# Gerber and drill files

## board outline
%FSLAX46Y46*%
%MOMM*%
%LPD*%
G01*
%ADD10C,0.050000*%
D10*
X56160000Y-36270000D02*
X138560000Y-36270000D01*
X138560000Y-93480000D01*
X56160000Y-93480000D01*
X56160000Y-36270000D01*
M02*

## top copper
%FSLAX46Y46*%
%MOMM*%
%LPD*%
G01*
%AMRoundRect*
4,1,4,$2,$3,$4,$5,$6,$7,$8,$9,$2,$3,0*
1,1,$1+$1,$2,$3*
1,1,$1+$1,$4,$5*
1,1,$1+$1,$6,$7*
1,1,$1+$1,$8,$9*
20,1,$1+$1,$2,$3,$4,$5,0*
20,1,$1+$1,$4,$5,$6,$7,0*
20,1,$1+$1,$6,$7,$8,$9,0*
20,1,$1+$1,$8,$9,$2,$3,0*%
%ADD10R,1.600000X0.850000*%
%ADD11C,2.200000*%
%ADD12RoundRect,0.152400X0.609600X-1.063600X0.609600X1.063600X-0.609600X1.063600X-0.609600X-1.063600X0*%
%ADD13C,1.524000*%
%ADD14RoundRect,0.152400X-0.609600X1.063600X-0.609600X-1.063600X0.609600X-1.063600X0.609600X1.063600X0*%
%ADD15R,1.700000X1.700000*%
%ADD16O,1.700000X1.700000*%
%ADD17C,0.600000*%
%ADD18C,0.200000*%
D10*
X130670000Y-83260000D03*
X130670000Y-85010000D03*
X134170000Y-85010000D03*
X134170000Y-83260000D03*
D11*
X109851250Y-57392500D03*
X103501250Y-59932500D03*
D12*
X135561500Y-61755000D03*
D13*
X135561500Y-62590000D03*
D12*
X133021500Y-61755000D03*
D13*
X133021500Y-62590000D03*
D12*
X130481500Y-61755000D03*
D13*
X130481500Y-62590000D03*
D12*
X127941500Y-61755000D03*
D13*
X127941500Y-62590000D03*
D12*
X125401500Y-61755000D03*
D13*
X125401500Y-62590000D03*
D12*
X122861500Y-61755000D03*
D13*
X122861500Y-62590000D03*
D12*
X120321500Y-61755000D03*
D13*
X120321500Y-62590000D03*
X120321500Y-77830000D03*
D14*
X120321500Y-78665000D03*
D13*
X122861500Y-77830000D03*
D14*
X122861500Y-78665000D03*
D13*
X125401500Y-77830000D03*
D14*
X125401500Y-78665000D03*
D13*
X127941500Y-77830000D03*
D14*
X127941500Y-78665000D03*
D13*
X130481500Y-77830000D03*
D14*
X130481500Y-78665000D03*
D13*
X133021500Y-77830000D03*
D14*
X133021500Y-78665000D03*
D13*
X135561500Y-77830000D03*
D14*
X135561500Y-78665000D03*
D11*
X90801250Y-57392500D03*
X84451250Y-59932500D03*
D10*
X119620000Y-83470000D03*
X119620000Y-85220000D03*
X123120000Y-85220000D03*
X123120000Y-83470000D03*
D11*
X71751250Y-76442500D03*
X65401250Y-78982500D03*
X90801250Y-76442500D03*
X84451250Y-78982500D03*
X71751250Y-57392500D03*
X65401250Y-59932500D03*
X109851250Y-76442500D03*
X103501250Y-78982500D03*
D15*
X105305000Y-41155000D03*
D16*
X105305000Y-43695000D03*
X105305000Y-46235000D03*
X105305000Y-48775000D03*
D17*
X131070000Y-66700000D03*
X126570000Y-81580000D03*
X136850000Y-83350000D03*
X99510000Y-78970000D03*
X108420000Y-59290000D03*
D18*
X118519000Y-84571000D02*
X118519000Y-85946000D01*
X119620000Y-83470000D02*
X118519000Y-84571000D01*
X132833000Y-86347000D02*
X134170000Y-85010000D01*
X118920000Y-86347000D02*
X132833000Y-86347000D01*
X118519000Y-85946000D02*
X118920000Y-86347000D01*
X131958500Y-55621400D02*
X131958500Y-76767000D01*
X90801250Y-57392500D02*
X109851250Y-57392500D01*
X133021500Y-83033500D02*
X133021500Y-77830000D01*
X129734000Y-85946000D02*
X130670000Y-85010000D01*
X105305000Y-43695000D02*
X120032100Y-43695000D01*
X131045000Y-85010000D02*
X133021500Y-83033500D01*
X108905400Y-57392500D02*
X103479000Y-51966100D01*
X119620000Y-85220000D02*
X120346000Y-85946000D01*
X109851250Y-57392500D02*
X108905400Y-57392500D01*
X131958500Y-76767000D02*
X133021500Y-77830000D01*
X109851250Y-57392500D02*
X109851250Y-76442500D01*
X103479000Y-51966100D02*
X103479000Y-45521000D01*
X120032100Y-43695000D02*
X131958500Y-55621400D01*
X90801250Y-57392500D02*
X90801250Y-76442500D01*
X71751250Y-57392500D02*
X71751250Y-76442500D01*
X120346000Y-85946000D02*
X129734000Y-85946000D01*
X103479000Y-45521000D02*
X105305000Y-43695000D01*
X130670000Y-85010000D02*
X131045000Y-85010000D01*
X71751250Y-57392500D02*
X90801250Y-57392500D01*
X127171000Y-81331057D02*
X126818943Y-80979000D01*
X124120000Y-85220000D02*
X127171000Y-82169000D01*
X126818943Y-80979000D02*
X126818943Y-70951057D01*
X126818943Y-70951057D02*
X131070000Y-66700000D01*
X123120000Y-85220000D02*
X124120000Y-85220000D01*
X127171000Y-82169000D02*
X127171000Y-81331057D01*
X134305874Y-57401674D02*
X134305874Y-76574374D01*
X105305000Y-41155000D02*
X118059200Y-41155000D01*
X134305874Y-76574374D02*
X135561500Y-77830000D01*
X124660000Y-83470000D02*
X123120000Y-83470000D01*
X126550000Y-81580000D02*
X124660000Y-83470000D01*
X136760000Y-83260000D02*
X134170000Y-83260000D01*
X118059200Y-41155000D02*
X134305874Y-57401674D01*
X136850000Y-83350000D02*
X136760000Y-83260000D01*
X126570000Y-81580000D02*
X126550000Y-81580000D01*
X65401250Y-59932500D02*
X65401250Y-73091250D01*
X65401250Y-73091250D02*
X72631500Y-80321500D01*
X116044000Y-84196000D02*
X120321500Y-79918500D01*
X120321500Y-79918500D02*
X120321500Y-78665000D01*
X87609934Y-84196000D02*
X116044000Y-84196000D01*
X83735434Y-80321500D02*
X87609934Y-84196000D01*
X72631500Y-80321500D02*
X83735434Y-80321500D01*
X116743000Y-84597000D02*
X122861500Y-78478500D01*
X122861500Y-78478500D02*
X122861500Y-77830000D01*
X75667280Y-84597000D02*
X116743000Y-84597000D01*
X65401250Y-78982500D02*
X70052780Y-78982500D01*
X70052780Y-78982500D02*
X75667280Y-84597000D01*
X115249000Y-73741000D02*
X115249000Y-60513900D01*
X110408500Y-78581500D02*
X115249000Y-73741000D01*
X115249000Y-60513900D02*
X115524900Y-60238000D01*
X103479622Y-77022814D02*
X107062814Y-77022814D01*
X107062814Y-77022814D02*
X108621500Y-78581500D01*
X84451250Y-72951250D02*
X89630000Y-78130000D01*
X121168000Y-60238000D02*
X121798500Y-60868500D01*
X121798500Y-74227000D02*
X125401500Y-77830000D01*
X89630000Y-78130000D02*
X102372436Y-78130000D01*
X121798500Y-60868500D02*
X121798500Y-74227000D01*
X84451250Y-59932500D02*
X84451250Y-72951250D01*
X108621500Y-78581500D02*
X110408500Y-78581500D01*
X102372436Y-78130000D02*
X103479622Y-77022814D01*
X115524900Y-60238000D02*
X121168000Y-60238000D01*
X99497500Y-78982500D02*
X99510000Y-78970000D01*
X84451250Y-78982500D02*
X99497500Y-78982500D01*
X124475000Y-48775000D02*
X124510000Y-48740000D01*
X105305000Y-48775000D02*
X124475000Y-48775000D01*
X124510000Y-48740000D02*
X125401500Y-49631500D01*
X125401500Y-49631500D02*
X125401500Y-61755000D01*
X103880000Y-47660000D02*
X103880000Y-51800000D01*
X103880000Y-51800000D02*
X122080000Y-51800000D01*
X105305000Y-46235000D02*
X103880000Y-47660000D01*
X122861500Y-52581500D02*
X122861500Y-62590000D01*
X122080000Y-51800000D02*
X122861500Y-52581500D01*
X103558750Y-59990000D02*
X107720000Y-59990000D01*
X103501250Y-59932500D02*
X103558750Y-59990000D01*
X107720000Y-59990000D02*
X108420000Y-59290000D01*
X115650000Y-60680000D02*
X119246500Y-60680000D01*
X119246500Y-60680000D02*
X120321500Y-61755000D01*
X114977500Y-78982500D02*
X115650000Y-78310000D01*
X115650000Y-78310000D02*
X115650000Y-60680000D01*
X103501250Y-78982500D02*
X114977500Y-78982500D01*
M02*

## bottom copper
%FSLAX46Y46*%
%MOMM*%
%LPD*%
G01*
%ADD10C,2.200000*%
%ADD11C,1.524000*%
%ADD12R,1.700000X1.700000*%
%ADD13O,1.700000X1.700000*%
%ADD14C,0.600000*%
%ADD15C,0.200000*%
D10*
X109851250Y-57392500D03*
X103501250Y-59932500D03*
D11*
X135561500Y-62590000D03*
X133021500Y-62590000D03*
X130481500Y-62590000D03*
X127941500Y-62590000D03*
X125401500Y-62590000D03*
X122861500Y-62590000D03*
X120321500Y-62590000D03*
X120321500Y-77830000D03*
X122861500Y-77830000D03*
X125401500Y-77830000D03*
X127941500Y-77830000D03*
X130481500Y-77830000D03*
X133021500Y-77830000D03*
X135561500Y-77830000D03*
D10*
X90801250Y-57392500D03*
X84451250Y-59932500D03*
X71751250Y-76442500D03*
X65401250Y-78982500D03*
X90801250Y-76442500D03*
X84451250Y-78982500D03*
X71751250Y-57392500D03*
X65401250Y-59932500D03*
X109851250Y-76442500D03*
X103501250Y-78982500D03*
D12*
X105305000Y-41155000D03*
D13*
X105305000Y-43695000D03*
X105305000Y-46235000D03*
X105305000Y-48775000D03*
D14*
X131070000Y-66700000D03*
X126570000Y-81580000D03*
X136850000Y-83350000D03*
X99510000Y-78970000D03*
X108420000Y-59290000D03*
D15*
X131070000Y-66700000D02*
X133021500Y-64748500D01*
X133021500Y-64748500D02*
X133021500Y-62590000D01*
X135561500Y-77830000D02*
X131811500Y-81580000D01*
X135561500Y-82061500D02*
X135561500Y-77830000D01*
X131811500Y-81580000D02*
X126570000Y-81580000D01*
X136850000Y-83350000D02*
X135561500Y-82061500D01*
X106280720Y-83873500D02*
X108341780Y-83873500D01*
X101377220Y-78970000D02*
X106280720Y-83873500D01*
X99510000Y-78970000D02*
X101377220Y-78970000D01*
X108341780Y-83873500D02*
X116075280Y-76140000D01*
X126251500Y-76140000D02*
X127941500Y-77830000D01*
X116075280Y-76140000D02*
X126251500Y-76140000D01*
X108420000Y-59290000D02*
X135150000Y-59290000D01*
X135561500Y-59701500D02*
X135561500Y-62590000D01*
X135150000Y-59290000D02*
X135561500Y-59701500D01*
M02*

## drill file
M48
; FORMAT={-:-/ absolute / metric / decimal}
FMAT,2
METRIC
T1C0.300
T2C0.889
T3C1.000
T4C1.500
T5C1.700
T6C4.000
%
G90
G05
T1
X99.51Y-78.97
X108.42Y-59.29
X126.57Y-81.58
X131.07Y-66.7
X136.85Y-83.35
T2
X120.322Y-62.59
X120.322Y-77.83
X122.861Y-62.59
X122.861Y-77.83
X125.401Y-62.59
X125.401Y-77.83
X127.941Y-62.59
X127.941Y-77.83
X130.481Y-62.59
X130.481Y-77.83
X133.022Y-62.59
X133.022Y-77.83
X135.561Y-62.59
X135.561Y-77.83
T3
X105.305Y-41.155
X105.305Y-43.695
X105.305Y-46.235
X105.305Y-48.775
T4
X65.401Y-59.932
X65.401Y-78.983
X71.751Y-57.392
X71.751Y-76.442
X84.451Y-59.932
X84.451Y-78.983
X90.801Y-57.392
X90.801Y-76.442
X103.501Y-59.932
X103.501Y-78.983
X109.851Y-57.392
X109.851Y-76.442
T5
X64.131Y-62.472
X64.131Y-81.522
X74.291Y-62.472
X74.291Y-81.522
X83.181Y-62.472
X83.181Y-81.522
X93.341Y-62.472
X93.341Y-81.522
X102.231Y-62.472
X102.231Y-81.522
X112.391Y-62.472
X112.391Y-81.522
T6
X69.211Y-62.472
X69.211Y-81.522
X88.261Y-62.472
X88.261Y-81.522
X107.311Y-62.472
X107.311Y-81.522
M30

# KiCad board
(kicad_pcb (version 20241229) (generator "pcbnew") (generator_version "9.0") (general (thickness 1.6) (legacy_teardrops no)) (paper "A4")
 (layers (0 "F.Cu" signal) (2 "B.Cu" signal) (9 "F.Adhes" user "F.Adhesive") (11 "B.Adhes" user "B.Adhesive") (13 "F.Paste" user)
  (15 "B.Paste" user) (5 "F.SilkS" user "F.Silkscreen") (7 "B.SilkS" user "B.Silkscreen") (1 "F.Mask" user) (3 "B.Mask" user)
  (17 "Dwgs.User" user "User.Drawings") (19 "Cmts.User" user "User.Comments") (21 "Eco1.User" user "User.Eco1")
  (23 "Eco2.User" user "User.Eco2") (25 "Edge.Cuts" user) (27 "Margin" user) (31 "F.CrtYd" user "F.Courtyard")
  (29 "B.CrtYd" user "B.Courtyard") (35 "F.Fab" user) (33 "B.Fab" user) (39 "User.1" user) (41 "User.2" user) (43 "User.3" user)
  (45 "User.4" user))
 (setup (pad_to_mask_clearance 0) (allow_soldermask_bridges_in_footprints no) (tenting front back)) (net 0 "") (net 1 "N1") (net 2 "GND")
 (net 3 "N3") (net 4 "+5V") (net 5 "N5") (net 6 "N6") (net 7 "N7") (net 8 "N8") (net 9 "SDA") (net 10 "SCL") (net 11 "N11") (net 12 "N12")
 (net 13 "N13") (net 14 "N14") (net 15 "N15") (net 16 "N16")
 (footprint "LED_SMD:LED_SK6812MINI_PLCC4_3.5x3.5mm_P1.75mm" (layer "F.Cu") (at 132.42 84.135)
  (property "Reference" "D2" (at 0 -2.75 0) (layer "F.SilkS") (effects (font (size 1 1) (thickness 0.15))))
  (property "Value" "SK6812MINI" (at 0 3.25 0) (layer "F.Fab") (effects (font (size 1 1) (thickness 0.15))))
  (pad "1" smd rect (at -1.75 -0.875) (size 1.6 0.85) (layers "F.Cu" "F.Mask" "F.Paste") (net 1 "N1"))
  (pad "2" smd rect (at -1.75 0.875) (size 1.6 0.85) (layers "F.Cu" "F.Mask" "F.Paste") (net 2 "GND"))
  (pad "3" smd rect (at 1.75 0.875) (size 1.6 0.85) (layers "F.Cu" "F.Mask" "F.Paste") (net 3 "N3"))
  (pad "4" smd rect (at 1.75 -0.875) (size 1.6 0.85) (layers "F.Cu" "F.Mask" "F.Paste") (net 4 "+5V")))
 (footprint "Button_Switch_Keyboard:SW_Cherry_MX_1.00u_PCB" (layer "F.Cu") (at 109.85125 57.3925)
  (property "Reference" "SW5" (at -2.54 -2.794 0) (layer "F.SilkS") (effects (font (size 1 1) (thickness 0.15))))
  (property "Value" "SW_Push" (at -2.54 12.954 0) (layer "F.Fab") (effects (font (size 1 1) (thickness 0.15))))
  (pad "" np_thru_hole circle (at -7.62 5.08) (size 1.7 1.7) (drill 1.7) (layers "*.Cu" "*.Mask"))
  (pad "" np_thru_hole circle (at -2.54 5.08) (size 4 4) (drill 4) (layers "*.Cu" "*.Mask"))
  (pad "" np_thru_hole circle (at 2.54 5.08) (size 1.7 1.7) (drill 1.7) (layers "*.Cu" "*.Mask"))
  (pad "1" thru_hole circle (at 0 0) (size 2.2 2.2) (drill 1.5) (layers "*.Cu" "*.Mask") (remove_unused_layers no) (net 2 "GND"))
  (pad "2" thru_hole circle (at -6.35 2.54) (size 2.2 2.2) (drill 1.5) (layers "*.Cu" "*.Mask") (remove_unused_layers no) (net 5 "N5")))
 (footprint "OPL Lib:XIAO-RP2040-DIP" (layer "F.Cu") (at 127.9415 70.21 -90)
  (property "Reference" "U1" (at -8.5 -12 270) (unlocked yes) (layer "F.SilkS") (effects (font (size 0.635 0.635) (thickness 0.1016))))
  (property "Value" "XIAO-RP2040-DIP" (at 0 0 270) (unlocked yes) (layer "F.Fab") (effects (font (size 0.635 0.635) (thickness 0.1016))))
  (pad "1" smd roundrect (at -8.455 -7.62 90) (size 2.432 1.524) (layers "F.Cu" "F.Mask") (roundrect_rratio 0.1) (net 5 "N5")
   (thermal_bridge_angle 45))
  (pad "1" thru_hole circle (at -7.62 -7.62 90) (size 1.524 1.524) (drill 0.889) (layers "*.Cu" "*.Mask") (remove_unused_layers no)
   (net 5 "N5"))
  (pad "2" smd roundrect (at -8.455 -5.08 90) (size 2.432 1.524) (layers "F.Cu" "F.Mask") (roundrect_rratio 0.1) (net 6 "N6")
   (thermal_bridge_angle 45))
  (pad "2" thru_hole circle (at -7.62 -5.08 90) (size 1.524 1.524) (drill 0.889) (layers "*.Cu" "*.Mask") (remove_unused_layers no)
   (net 6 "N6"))
  (pad "3" smd roundrect (at -8.455 -2.54 90) (size 2.432 1.524) (layers "F.Cu" "F.Mask") (roundrect_rratio 0.1) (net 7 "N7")
   (thermal_bridge_angle 45))
  (pad "3" thru_hole circle (at -7.62 -2.54 90) (size 1.524 1.524) (drill 0.889) (layers "*.Cu" "*.Mask") (remove_unused_layers no)
   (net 7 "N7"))
  (pad "4" smd roundrect (at -8.455 0 90) (size 2.432 1.524) (layers "F.Cu" "F.Mask") (roundrect_rratio 0.1) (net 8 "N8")
   (thermal_bridge_angle 45))
  (pad "4" thru_hole circle (at -7.62 0 90) (size 1.524 1.524) (drill 0.889) (layers "*.Cu" "*.Mask") (remove_unused_layers no) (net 8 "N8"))
  (pad "5" smd roundrect (at -8.455 2.54 90) (size 2.432 1.524) (layers "F.Cu" "F.Mask") (roundrect_rratio 0.1) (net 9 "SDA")
   (thermal_bridge_angle 45))
  (pad "5" thru_hole circle (at -7.62 2.54 90) (size 1.524 1.524) (drill 0.889) (layers "*.Cu" "*.Mask") (remove_unused_layers no)
   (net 9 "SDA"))
  (pad "6" smd roundrect (at -8.455 5.08 90) (size 2.432 1.524) (layers "F.Cu" "F.Mask") (roundrect_rratio 0.1) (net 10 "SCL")
   (thermal_bridge_angle 45))
  (pad "6" thru_hole circle (at -7.62 5.08 90) (size 1.524 1.524) (drill 0.889) (layers "*.Cu" "*.Mask") (remove_unused_layers no)
   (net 10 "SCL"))
  (pad "7" smd roundrect (at -8.455 7.62 90) (size 2.432 1.524) (layers "F.Cu" "F.Mask") (roundrect_rratio 0.1) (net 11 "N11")
   (thermal_bridge_angle 45))
  (pad "7" thru_hole circle (at -7.62 7.62 90) (size 1.524 1.524) (drill 0.889) (layers "*.Cu" "*.Mask") (remove_unused_layers no)
   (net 11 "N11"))
  (pad "8" thru_hole circle (at 7.62 7.62 270) (size 1.524 1.524) (drill 0.889) (layers "*.Cu" "*.Mask") (remove_unused_layers no)
   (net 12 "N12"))
  (pad "8" smd roundrect (at 8.455 7.62 270) (size 2.432 1.524) (layers "F.Cu" "F.Mask") (roundrect_rratio 0.1) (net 12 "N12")
   (thermal_bridge_angle 45))
  (pad "9" thru_hole circle (at 7.62 5.08 270) (size 1.524 1.524) (drill 0.889) (layers "*.Cu" "*.Mask") (remove_unused_layers no)
   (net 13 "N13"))
  (pad "9" smd roundrect (at 8.455 5.08 270) (size 2.432 1.524) (layers "F.Cu" "F.Mask") (roundrect_rratio 0.1) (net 13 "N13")
   (thermal_bridge_angle 45))
  (pad "10" thru_hole circle (at 7.62 2.54 270) (size 1.524 1.524) (drill 0.889) (layers "*.Cu" "*.Mask") (remove_unused_layers no)
   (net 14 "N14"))
  (pad "10" smd roundrect (at 8.455 2.54 270) (size 2.432 1.524) (layers "F.Cu" "F.Mask") (roundrect_rratio 0.1) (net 14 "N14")
   (thermal_bridge_angle 45))
  (pad "11" thru_hole circle (at 7.62 0 270) (size 1.524 1.524) (drill 0.889) (layers "*.Cu" "*.Mask") (remove_unused_layers no)
   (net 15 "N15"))
  (pad "11" smd roundrect (at 8.455 0 270) (size 2.432 1.524) (layers "F.Cu" "F.Mask") (roundrect_rratio 0.1) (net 15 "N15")
   (thermal_bridge_angle 45))
  (pad "12" thru_hole circle (at 7.62 -2.54 270) (size 1.524 1.524) (drill 0.889) (layers "*.Cu" "*.Mask") (remove_unused_layers no)
   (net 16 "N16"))
  (pad "12" smd roundrect (at 8.455 -2.54 270) (size 2.432 1.524) (layers "F.Cu" "F.Mask") (roundrect_rratio 0.1) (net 16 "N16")
   (thermal_bridge_angle 45))
  (pad "13" thru_hole circle (at 7.62 -5.08 270) (size 1.524 1.524) (drill 0.889) (layers "*.Cu" "*.Mask") (remove_unused_layers no)
   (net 2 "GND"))
  (pad "13" smd roundrect (at 8.455 -5.08 270) (size 2.432 1.524) (layers "F.Cu" "F.Mask") (roundrect_rratio 0.1) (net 2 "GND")
   (thermal_bridge_angle 45))
  (pad "14" thru_hole circle (at 7.62 -7.62 270) (size 1.524 1.524) (drill 0.889) (layers "*.Cu" "*.Mask") (remove_unused_layers no)
   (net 4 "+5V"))
  (pad "14" smd roundrect (at 8.455 -7.62 270) (size 2.432 1.524) (layers "F.Cu" "F.Mask") (roundrect_rratio 0.1) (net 4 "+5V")
   (thermal_bridge_angle 45)))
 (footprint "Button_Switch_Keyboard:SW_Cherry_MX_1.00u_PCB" (layer "F.Cu") (at 90.80125 57.3925)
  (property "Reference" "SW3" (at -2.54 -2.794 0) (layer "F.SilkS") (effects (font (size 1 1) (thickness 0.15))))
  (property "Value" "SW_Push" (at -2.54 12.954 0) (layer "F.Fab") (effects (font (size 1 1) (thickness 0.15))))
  (pad "" np_thru_hole circle (at -7.62 5.08) (size 1.7 1.7) (drill 1.7) (layers "*.Cu" "*.Mask"))
  (pad "" np_thru_hole circle (at -2.54 5.08) (size 4 4) (drill 4) (layers "*.Cu" "*.Mask"))
  (pad "" np_thru_hole circle (at 2.54 5.08) (size 1.7 1.7) (drill 1.7) (layers "*.Cu" "*.Mask"))
  (pad "1" thru_hole circle (at 0 0) (size 2.2 2.2) (drill 1.5) (layers "*.Cu" "*.Mask") (remove_unused_layers no) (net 2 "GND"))
  (pad "2" thru_hole circle (at -6.35 2.54) (size 2.2 2.2) (drill 1.5) (layers "*.Cu" "*.Mask") (remove_unused_layers no) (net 14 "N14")))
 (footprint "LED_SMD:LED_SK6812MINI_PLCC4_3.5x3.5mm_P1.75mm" (layer "F.Cu") (at 121.37 84.345)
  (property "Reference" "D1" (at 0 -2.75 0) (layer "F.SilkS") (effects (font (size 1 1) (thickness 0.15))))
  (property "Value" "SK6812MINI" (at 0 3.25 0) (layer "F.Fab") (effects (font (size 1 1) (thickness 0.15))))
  (pad "1" smd rect (at -1.75 -0.875) (size 1.6 0.85) (layers "F.Cu" "F.Mask" "F.Paste") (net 3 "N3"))
  (pad "2" smd rect (at -1.75 0.875) (size 1.6 0.85) (layers "F.Cu" "F.Mask" "F.Paste") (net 2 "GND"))
  (pad "3" smd rect (at 1.75 0.875) (size 1.6 0.85) (layers "F.Cu" "F.Mask" "F.Paste") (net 6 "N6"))
  (pad "4" smd rect (at 1.75 -0.875) (size 1.6 0.85) (layers "F.Cu" "F.Mask" "F.Paste") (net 4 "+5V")))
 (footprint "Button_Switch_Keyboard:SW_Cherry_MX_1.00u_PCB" (layer "F.Cu") (at 71.75125 76.4425)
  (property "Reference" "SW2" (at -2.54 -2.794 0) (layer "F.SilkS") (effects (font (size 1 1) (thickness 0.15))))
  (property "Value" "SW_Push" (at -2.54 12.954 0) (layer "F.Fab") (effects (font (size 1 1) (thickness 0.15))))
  (pad "" np_thru_hole circle (at -7.62 5.08) (size 1.7 1.7) (drill 1.7) (layers "*.Cu" "*.Mask"))
  (pad "" np_thru_hole circle (at -2.54 5.08) (size 4 4) (drill 4) (layers "*.Cu" "*.Mask"))
  (pad "" np_thru_hole circle (at 2.54 5.08) (size 1.7 1.7) (drill 1.7) (layers "*.Cu" "*.Mask"))
  (pad "1" thru_hole circle (at 0 0) (size 2.2 2.2) (drill 1.5) (layers "*.Cu" "*.Mask") (remove_unused_layers no) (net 2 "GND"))
  (pad "2" thru_hole circle (at -6.35 2.54) (size 2.2 2.2) (drill 1.5) (layers "*.Cu" "*.Mask") (remove_unused_layers no) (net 13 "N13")))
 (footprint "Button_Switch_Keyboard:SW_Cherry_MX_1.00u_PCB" (layer "F.Cu") (at 90.80125 76.4425)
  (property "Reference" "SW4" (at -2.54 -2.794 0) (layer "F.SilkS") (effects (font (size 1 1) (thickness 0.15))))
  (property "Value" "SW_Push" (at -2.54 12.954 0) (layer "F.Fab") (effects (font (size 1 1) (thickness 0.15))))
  (pad "" np_thru_hole circle (at -7.62 5.08) (size 1.7 1.7) (drill 1.7) (layers "*.Cu" "*.Mask"))
  (pad "" np_thru_hole circle (at -2.54 5.08) (size 4 4) (drill 4) (layers "*.Cu" "*.Mask"))
  (pad "" np_thru_hole circle (at 2.54 5.08) (size 1.7 1.7) (drill 1.7) (layers "*.Cu" "*.Mask"))
  (pad "1" thru_hole circle (at 0 0) (size 2.2 2.2) (drill 1.5) (layers "*.Cu" "*.Mask") (remove_unused_layers no) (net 2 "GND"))
  (pad "2" thru_hole circle (at -6.35 2.54) (size 2.2 2.2) (drill 1.5) (layers "*.Cu" "*.Mask") (remove_unused_layers no) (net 15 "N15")))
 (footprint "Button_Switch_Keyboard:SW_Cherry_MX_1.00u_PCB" (layer "F.Cu") (at 71.75125 57.3925)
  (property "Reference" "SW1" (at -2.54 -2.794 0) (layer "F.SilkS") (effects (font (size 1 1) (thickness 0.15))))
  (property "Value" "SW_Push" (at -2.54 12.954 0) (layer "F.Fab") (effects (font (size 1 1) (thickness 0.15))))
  (pad "" np_thru_hole circle (at -7.62 5.08) (size 1.7 1.7) (drill 1.7) (layers "*.Cu" "*.Mask"))
  (pad "" np_thru_hole circle (at -2.54 5.08) (size 4 4) (drill 4) (layers "*.Cu" "*.Mask"))
  (pad "" np_thru_hole circle (at 2.54 5.08) (size 1.7 1.7) (drill 1.7) (layers "*.Cu" "*.Mask"))
  (pad "1" thru_hole circle (at 0 0) (size 2.2 2.2) (drill 1.5) (layers "*.Cu" "*.Mask") (remove_unused_layers no) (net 2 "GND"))
  (pad "2" thru_hole circle (at -6.35 2.54) (size 2.2 2.2) (drill 1.5) (layers "*.Cu" "*.Mask") (remove_unused_layers no) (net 12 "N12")))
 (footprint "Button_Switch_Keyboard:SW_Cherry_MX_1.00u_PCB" (layer "F.Cu") (at 109.85125 76.4425)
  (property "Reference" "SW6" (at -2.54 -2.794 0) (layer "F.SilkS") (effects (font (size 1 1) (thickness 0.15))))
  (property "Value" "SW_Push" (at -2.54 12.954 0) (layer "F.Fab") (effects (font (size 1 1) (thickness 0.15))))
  (pad "" np_thru_hole circle (at -7.62 5.08) (size 1.7 1.7) (drill 1.7) (layers "*.Cu" "*.Mask"))
  (pad "" np_thru_hole circle (at -2.54 5.08) (size 4 4) (drill 4) (layers "*.Cu" "*.Mask"))
  (pad "" np_thru_hole circle (at 2.54 5.08) (size 1.7 1.7) (drill 1.7) (layers "*.Cu" "*.Mask"))
  (pad "1" thru_hole circle (at 0 0) (size 2.2 2.2) (drill 1.5) (layers "*.Cu" "*.Mask") (remove_unused_layers no) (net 2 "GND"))
  (pad "2" thru_hole circle (at -6.35 2.54) (size 2.2 2.2) (drill 1.5) (layers "*.Cu" "*.Mask") (remove_unused_layers no) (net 11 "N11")))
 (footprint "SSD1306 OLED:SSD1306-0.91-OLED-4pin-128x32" (layer "F.Cu") (at 68.805 38.965)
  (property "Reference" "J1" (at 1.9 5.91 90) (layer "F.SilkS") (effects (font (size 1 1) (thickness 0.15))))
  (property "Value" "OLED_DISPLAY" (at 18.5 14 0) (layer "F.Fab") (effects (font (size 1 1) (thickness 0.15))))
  (pad "1" thru_hole rect (at 36.5 2.19) (size 1.7 1.7) (drill 1) (layers "*.Cu" "*.Mask") (remove_unused_layers no) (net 4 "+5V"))
  (pad "2" thru_hole oval (at 36.5 4.73) (size 1.7 1.7) (drill 1) (layers "*.Cu" "*.Mask") (remove_unused_layers no) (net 2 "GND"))
  (pad "3" thru_hole oval (at 36.5 7.27) (size 1.7 1.7) (drill 1) (layers "*.Cu" "*.Mask") (remove_unused_layers no) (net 10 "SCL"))
  (pad "4" thru_hole oval (at 36.5 9.81) (size 1.7 1.7) (drill 1) (layers "*.Cu" "*.Mask") (remove_unused_layers no) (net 9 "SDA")))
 (gr_rect (start 56.16 36.27) (end 138.56 93.48) (stroke (width 0.05) (type default)) (fill no) (layer "Edge.Cuts"))
 (segment (start 118.519 84.571) (end 118.519 85.946) (width 0.2) (layer "F.Cu") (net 3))
 (segment (start 119.62 83.47) (end 118.519 84.571) (width 0.2) (layer "F.Cu") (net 3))
 (segment (start 132.833 86.347) (end 134.17 85.01) (width 0.2) (layer "F.Cu") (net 3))
 (segment (start 118.92 86.347) (end 132.833 86.347) (width 0.2) (layer "F.Cu") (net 3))
 (segment (start 118.519 85.946) (end 118.92 86.347) (width 0.2) (layer "F.Cu") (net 3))
 (segment (start 131.9585 55.6214) (end 131.9585 76.767) (width 0.2) (layer "F.Cu") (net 2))
 (segment (start 90.80125 57.3925) (end 109.85125 57.3925) (width 0.2) (layer "F.Cu") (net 2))
 (segment (start 133.0215 83.0335) (end 133.0215 77.83) (width 0.2) (layer "F.Cu") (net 2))
 (segment (start 129.734 85.946) (end 130.67 85.01) (width 0.2) (layer "F.Cu") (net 2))
 (segment (start 105.305 43.695) (end 120.0321 43.695) (width 0.2) (layer "F.Cu") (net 2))
 (segment (start 131.045 85.01) (end 133.0215 83.0335) (width 0.2) (layer "F.Cu") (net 2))
 (segment (start 108.9054 57.3925) (end 103.479 51.9661) (width 0.2) (layer "F.Cu") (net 2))
 (segment (start 119.62 85.22) (end 120.346 85.946) (width 0.2) (layer "F.Cu") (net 2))
 (segment (start 109.85125 57.3925) (end 108.9054 57.3925) (width 0.2) (layer "F.Cu") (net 2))
 (segment (start 131.9585 76.767) (end 133.0215 77.83) (width 0.2) (layer "F.Cu") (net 2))
 (segment (start 109.85125 57.3925) (end 109.85125 76.4425) (width 0.2) (layer "F.Cu") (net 2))
 (segment (start 103.479 51.9661) (end 103.479 45.521) (width 0.2) (layer "F.Cu") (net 2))
 (segment (start 120.0321 43.695) (end 131.9585 55.6214) (width 0.2) (layer "F.Cu") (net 2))
 (segment (start 90.80125 57.3925) (end 90.80125 76.4425) (width 0.2) (layer "F.Cu") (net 2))
 (segment (start 71.75125 57.3925) (end 71.75125 76.4425) (width 0.2) (layer "F.Cu") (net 2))
 (segment (start 120.346 85.946) (end 129.734 85.946) (width 0.2) (layer "F.Cu") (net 2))
 (segment (start 103.479 45.521) (end 105.305 43.695) (width 0.2) (layer "F.Cu") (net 2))
 (segment (start 130.67 85.01) (end 131.045 85.01) (width 0.2) (layer "F.Cu") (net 2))
 (segment (start 71.75125 57.3925) (end 90.80125 57.3925) (width 0.2) (layer "F.Cu") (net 2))
 (segment (start 127.171 81.331057) (end 126.818943 80.979) (width 0.2) (layer "F.Cu") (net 6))
 (segment (start 124.12 85.22) (end 127.171 82.169) (width 0.2) (layer "F.Cu") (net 6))
 (segment (start 126.818943 80.979) (end 126.818943 70.951057) (width 0.2) (layer "F.Cu") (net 6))
 (segment (start 126.818943 70.951057) (end 131.07 66.7) (width 0.2) (layer "F.Cu") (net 6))
 (segment (start 123.12 85.22) (end 124.12 85.22) (width 0.2) (layer "F.Cu") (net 6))
 (segment (start 127.171 82.169) (end 127.171 81.331057) (width 0.2) (layer "F.Cu") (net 6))
 (via (at 131.07 66.7) (size 0.6) (drill 0.3) (layers "F.Cu" "B.Cu") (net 6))
 (segment (start 131.07 66.7) (end 133.0215 64.7485) (width 0.2) (layer "B.Cu") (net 6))
 (segment (start 133.0215 64.7485) (end 133.0215 62.59) (width 0.2) (layer "B.Cu") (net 6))
 (segment (start 134.305874 57.401674) (end 134.305874 76.574374) (width 0.2) (layer "F.Cu") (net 4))
 (segment (start 105.305 41.155) (end 118.0592 41.155) (width 0.2) (layer "F.Cu") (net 4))
 (segment (start 134.305874 76.574374) (end 135.5615 77.83) (width 0.2) (layer "F.Cu") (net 4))
 (segment (start 124.66 83.47) (end 123.12 83.47) (width 0.2) (layer "F.Cu") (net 4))
 (segment (start 126.55 81.58) (end 124.66 83.47) (width 0.2) (layer "F.Cu") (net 4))
 (segment (start 136.76 83.26) (end 134.17 83.26) (width 0.2) (layer "F.Cu") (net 4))
 (segment (start 118.0592 41.155) (end 134.305874 57.401674) (width 0.2) (layer "F.Cu") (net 4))
 (segment (start 136.85 83.35) (end 136.76 83.26) (width 0.2) (layer "F.Cu") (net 4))
 (segment (start 126.57 81.58) (end 126.55 81.58) (width 0.2) (layer "F.Cu") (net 4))
 (via (at 126.57 81.58) (size 0.6) (drill 0.3) (layers "F.Cu" "B.Cu") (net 4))
 (via (at 136.85 83.35) (size 0.6) (drill 0.3) (layers "F.Cu" "B.Cu") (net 4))
 (segment (start 135.5615 77.83) (end 131.8115 81.58) (width 0.2) (layer "B.Cu") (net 4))
 (segment (start 135.5615 82.0615) (end 135.5615 77.83) (width 0.2) (layer "B.Cu") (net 4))
 (segment (start 131.8115 81.58) (end 126.57 81.58) (width 0.2) (layer "B.Cu") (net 4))
 (segment (start 136.85 83.35) (end 135.5615 82.0615) (width 0.2) (layer "B.Cu") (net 4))
 (segment (start 65.40125 59.9325) (end 65.40125 73.09125) (width 0.2) (layer "F.Cu") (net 12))
 (segment (start 65.40125 73.09125) (end 72.6315 80.3215) (width 0.2) (layer "F.Cu") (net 12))
 (segment (start 116.044 84.196) (end 120.3215 79.9185) (width 0.2) (layer "F.Cu") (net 12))
 (segment (start 120.3215 79.9185) (end 120.3215 78.665) (width 0.2) (layer "F.Cu") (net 12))
 (segment (start 87.609934 84.196) (end 116.044 84.196) (width 0.2) (layer "F.Cu") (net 12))
 (segment (start 83.735434 80.3215) (end 87.609934 84.196) (width 0.2) (layer "F.Cu") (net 12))
 (segment (start 72.6315 80.3215) (end 83.735434 80.3215) (width 0.2) (layer "F.Cu") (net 12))
 (segment (start 116.743 84.597) (end 122.8615 78.4785) (width 0.2) (layer "F.Cu") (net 13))
 (segment (start 122.8615 78.4785) (end 122.8615 77.83) (width 0.2) (layer "F.Cu") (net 13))
 (segment (start 75.66728 84.597) (end 116.743 84.597) (width 0.2) (layer "F.Cu") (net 13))
 (segment (start 65.40125 78.9825) (end 70.05278 78.9825) (width 0.2) (layer "F.Cu") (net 13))
 (segment (start 70.05278 78.9825) (end 75.66728 84.597) (width 0.2) (layer "F.Cu") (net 13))
 (segment (start 115.249 73.741) (end 115.249 60.5139) (width 0.2) (layer "F.Cu") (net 14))
 (segment (start 110.4085 78.5815) (end 115.249 73.741) (width 0.2) (layer "F.Cu") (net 14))
 (segment (start 115.249 60.5139) (end 115.5249 60.238) (width 0.2) (layer "F.Cu") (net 14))
 (segment (start 103.479622 77.022814) (end 107.062814 77.022814) (width 0.2) (layer "F.Cu") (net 14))
 (segment (start 107.062814 77.022814) (end 108.6215 78.5815) (width 0.2) (layer "F.Cu") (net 14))
 (segment (start 84.45125 72.95125) (end 89.63 78.13) (width 0.2) (layer "F.Cu") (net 14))
 (segment (start 121.168 60.238) (end 121.7985 60.8685) (width 0.2) (layer "F.Cu") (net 14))
 (segment (start 121.7985 74.227) (end 125.4015 77.83) (width 0.2) (layer "F.Cu") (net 14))
 (segment (start 89.63 78.13) (end 102.372436 78.13) (width 0.2) (layer "F.Cu") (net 14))
 (segment (start 121.7985 60.8685) (end 121.7985 74.227) (width 0.2) (layer "F.Cu") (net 14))
 (segment (start 84.45125 59.9325) (end 84.45125 72.95125) (width 0.2) (layer "F.Cu") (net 14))
 (segment (start 108.6215 78.5815) (end 110.4085 78.5815) (width 0.2) (layer "F.Cu") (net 14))
 (segment (start 102.372436 78.13) (end 103.479622 77.022814) (width 0.2) (layer "F.Cu") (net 14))
 (segment (start 115.5249 60.238) (end 121.168 60.238) (width 0.2) (layer "F.Cu") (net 14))
 (segment (start 99.4975 78.9825) (end 99.51 78.97) (width 0.2) (layer "F.Cu") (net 15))
 (segment (start 84.45125 78.9825) (end 99.4975 78.9825) (width 0.2) (layer "F.Cu") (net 15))
 (via (at 99.51 78.97) (size 0.6) (drill 0.3) (layers "F.Cu" "B.Cu") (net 15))
 (segment (start 106.28072 83.8735) (end 108.34178 83.8735) (width 0.2) (layer "B.Cu") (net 15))
 (segment (start 101.37722 78.97) (end 106.28072 83.8735) (width 0.2) (layer "B.Cu") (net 15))
 (segment (start 99.51 78.97) (end 101.37722 78.97) (width 0.2) (layer "B.Cu") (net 15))
 (segment (start 108.34178 83.8735) (end 116.07528 76.14) (width 0.2) (layer "B.Cu") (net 15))
 (segment (start 126.2515 76.14) (end 127.9415 77.83) (width 0.2) (layer "B.Cu") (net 15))
 (segment (start 116.07528 76.14) (end 126.2515 76.14) (width 0.2) (layer "B.Cu") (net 15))
 (segment (start 124.475 48.775) (end 124.51 48.74) (width 0.2) (layer "F.Cu") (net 9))
 (segment (start 105.305 48.775) (end 124.475 48.775) (width 0.2) (layer "F.Cu") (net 9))
 (segment (start 124.51 48.74) (end 125.4015 49.6315) (width 0.2) (layer "F.Cu") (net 9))
 (segment (start 125.4015 49.6315) (end 125.4015 61.755) (width 0.2) (layer "F.Cu") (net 9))
 (segment (start 103.88 47.66) (end 103.88 51.8) (width 0.2) (layer "F.Cu") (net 10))
 (segment (start 103.88 51.8) (end 122.08 51.8) (width 0.2) (layer "F.Cu") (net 10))
 (segment (start 105.305 46.235) (end 103.88 47.66) (width 0.2) (layer "F.Cu") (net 10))
 (segment (start 122.8615 52.5815) (end 122.8615 62.59) (width 0.2) (layer "F.Cu") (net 10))
 (segment (start 122.08 51.8) (end 122.8615 52.5815) (width 0.2) (layer "F.Cu") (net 10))
 (segment (start 103.55875 59.99) (end 107.72 59.99) (width 0.2) (layer "F.Cu") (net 5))
 (segment (start 103.50125 59.9325) (end 103.55875 59.99) (width 0.2) (layer "F.Cu") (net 5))
 (segment (start 107.72 59.99) (end 108.42 59.29) (width 0.2) (layer "F.Cu") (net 5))
 (via (at 108.42 59.29) (size 0.6) (drill 0.3) (layers "F.Cu" "B.Cu") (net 5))
 (segment (start 108.42 59.29) (end 135.15 59.29) (width 0.2) (layer "B.Cu") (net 5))
 (segment (start 135.5615 59.7015) (end 135.5615 62.59) (width 0.2) (layer "B.Cu") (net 5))
 (segment (start 135.15 59.29) (end 135.5615 59.7015) (width 0.2) (layer "B.Cu") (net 5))
 (segment (start 115.65 60.68) (end 119.2465 60.68) (width 0.2) (layer "F.Cu") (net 11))
 (segment (start 119.2465 60.68) (end 120.3215 61.755) (width 0.2) (layer "F.Cu") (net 11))
 (segment (start 114.9775 78.9825) (end 115.65 78.31) (width 0.2) (layer "F.Cu") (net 11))
 (segment (start 115.65 78.31) (end 115.65 60.68) (width 0.2) (layer "F.Cu") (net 11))
 (segment (start 103.50125 78.9825) (end 114.9775 78.9825) (width 0.2) (layer "F.Cu") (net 11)))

